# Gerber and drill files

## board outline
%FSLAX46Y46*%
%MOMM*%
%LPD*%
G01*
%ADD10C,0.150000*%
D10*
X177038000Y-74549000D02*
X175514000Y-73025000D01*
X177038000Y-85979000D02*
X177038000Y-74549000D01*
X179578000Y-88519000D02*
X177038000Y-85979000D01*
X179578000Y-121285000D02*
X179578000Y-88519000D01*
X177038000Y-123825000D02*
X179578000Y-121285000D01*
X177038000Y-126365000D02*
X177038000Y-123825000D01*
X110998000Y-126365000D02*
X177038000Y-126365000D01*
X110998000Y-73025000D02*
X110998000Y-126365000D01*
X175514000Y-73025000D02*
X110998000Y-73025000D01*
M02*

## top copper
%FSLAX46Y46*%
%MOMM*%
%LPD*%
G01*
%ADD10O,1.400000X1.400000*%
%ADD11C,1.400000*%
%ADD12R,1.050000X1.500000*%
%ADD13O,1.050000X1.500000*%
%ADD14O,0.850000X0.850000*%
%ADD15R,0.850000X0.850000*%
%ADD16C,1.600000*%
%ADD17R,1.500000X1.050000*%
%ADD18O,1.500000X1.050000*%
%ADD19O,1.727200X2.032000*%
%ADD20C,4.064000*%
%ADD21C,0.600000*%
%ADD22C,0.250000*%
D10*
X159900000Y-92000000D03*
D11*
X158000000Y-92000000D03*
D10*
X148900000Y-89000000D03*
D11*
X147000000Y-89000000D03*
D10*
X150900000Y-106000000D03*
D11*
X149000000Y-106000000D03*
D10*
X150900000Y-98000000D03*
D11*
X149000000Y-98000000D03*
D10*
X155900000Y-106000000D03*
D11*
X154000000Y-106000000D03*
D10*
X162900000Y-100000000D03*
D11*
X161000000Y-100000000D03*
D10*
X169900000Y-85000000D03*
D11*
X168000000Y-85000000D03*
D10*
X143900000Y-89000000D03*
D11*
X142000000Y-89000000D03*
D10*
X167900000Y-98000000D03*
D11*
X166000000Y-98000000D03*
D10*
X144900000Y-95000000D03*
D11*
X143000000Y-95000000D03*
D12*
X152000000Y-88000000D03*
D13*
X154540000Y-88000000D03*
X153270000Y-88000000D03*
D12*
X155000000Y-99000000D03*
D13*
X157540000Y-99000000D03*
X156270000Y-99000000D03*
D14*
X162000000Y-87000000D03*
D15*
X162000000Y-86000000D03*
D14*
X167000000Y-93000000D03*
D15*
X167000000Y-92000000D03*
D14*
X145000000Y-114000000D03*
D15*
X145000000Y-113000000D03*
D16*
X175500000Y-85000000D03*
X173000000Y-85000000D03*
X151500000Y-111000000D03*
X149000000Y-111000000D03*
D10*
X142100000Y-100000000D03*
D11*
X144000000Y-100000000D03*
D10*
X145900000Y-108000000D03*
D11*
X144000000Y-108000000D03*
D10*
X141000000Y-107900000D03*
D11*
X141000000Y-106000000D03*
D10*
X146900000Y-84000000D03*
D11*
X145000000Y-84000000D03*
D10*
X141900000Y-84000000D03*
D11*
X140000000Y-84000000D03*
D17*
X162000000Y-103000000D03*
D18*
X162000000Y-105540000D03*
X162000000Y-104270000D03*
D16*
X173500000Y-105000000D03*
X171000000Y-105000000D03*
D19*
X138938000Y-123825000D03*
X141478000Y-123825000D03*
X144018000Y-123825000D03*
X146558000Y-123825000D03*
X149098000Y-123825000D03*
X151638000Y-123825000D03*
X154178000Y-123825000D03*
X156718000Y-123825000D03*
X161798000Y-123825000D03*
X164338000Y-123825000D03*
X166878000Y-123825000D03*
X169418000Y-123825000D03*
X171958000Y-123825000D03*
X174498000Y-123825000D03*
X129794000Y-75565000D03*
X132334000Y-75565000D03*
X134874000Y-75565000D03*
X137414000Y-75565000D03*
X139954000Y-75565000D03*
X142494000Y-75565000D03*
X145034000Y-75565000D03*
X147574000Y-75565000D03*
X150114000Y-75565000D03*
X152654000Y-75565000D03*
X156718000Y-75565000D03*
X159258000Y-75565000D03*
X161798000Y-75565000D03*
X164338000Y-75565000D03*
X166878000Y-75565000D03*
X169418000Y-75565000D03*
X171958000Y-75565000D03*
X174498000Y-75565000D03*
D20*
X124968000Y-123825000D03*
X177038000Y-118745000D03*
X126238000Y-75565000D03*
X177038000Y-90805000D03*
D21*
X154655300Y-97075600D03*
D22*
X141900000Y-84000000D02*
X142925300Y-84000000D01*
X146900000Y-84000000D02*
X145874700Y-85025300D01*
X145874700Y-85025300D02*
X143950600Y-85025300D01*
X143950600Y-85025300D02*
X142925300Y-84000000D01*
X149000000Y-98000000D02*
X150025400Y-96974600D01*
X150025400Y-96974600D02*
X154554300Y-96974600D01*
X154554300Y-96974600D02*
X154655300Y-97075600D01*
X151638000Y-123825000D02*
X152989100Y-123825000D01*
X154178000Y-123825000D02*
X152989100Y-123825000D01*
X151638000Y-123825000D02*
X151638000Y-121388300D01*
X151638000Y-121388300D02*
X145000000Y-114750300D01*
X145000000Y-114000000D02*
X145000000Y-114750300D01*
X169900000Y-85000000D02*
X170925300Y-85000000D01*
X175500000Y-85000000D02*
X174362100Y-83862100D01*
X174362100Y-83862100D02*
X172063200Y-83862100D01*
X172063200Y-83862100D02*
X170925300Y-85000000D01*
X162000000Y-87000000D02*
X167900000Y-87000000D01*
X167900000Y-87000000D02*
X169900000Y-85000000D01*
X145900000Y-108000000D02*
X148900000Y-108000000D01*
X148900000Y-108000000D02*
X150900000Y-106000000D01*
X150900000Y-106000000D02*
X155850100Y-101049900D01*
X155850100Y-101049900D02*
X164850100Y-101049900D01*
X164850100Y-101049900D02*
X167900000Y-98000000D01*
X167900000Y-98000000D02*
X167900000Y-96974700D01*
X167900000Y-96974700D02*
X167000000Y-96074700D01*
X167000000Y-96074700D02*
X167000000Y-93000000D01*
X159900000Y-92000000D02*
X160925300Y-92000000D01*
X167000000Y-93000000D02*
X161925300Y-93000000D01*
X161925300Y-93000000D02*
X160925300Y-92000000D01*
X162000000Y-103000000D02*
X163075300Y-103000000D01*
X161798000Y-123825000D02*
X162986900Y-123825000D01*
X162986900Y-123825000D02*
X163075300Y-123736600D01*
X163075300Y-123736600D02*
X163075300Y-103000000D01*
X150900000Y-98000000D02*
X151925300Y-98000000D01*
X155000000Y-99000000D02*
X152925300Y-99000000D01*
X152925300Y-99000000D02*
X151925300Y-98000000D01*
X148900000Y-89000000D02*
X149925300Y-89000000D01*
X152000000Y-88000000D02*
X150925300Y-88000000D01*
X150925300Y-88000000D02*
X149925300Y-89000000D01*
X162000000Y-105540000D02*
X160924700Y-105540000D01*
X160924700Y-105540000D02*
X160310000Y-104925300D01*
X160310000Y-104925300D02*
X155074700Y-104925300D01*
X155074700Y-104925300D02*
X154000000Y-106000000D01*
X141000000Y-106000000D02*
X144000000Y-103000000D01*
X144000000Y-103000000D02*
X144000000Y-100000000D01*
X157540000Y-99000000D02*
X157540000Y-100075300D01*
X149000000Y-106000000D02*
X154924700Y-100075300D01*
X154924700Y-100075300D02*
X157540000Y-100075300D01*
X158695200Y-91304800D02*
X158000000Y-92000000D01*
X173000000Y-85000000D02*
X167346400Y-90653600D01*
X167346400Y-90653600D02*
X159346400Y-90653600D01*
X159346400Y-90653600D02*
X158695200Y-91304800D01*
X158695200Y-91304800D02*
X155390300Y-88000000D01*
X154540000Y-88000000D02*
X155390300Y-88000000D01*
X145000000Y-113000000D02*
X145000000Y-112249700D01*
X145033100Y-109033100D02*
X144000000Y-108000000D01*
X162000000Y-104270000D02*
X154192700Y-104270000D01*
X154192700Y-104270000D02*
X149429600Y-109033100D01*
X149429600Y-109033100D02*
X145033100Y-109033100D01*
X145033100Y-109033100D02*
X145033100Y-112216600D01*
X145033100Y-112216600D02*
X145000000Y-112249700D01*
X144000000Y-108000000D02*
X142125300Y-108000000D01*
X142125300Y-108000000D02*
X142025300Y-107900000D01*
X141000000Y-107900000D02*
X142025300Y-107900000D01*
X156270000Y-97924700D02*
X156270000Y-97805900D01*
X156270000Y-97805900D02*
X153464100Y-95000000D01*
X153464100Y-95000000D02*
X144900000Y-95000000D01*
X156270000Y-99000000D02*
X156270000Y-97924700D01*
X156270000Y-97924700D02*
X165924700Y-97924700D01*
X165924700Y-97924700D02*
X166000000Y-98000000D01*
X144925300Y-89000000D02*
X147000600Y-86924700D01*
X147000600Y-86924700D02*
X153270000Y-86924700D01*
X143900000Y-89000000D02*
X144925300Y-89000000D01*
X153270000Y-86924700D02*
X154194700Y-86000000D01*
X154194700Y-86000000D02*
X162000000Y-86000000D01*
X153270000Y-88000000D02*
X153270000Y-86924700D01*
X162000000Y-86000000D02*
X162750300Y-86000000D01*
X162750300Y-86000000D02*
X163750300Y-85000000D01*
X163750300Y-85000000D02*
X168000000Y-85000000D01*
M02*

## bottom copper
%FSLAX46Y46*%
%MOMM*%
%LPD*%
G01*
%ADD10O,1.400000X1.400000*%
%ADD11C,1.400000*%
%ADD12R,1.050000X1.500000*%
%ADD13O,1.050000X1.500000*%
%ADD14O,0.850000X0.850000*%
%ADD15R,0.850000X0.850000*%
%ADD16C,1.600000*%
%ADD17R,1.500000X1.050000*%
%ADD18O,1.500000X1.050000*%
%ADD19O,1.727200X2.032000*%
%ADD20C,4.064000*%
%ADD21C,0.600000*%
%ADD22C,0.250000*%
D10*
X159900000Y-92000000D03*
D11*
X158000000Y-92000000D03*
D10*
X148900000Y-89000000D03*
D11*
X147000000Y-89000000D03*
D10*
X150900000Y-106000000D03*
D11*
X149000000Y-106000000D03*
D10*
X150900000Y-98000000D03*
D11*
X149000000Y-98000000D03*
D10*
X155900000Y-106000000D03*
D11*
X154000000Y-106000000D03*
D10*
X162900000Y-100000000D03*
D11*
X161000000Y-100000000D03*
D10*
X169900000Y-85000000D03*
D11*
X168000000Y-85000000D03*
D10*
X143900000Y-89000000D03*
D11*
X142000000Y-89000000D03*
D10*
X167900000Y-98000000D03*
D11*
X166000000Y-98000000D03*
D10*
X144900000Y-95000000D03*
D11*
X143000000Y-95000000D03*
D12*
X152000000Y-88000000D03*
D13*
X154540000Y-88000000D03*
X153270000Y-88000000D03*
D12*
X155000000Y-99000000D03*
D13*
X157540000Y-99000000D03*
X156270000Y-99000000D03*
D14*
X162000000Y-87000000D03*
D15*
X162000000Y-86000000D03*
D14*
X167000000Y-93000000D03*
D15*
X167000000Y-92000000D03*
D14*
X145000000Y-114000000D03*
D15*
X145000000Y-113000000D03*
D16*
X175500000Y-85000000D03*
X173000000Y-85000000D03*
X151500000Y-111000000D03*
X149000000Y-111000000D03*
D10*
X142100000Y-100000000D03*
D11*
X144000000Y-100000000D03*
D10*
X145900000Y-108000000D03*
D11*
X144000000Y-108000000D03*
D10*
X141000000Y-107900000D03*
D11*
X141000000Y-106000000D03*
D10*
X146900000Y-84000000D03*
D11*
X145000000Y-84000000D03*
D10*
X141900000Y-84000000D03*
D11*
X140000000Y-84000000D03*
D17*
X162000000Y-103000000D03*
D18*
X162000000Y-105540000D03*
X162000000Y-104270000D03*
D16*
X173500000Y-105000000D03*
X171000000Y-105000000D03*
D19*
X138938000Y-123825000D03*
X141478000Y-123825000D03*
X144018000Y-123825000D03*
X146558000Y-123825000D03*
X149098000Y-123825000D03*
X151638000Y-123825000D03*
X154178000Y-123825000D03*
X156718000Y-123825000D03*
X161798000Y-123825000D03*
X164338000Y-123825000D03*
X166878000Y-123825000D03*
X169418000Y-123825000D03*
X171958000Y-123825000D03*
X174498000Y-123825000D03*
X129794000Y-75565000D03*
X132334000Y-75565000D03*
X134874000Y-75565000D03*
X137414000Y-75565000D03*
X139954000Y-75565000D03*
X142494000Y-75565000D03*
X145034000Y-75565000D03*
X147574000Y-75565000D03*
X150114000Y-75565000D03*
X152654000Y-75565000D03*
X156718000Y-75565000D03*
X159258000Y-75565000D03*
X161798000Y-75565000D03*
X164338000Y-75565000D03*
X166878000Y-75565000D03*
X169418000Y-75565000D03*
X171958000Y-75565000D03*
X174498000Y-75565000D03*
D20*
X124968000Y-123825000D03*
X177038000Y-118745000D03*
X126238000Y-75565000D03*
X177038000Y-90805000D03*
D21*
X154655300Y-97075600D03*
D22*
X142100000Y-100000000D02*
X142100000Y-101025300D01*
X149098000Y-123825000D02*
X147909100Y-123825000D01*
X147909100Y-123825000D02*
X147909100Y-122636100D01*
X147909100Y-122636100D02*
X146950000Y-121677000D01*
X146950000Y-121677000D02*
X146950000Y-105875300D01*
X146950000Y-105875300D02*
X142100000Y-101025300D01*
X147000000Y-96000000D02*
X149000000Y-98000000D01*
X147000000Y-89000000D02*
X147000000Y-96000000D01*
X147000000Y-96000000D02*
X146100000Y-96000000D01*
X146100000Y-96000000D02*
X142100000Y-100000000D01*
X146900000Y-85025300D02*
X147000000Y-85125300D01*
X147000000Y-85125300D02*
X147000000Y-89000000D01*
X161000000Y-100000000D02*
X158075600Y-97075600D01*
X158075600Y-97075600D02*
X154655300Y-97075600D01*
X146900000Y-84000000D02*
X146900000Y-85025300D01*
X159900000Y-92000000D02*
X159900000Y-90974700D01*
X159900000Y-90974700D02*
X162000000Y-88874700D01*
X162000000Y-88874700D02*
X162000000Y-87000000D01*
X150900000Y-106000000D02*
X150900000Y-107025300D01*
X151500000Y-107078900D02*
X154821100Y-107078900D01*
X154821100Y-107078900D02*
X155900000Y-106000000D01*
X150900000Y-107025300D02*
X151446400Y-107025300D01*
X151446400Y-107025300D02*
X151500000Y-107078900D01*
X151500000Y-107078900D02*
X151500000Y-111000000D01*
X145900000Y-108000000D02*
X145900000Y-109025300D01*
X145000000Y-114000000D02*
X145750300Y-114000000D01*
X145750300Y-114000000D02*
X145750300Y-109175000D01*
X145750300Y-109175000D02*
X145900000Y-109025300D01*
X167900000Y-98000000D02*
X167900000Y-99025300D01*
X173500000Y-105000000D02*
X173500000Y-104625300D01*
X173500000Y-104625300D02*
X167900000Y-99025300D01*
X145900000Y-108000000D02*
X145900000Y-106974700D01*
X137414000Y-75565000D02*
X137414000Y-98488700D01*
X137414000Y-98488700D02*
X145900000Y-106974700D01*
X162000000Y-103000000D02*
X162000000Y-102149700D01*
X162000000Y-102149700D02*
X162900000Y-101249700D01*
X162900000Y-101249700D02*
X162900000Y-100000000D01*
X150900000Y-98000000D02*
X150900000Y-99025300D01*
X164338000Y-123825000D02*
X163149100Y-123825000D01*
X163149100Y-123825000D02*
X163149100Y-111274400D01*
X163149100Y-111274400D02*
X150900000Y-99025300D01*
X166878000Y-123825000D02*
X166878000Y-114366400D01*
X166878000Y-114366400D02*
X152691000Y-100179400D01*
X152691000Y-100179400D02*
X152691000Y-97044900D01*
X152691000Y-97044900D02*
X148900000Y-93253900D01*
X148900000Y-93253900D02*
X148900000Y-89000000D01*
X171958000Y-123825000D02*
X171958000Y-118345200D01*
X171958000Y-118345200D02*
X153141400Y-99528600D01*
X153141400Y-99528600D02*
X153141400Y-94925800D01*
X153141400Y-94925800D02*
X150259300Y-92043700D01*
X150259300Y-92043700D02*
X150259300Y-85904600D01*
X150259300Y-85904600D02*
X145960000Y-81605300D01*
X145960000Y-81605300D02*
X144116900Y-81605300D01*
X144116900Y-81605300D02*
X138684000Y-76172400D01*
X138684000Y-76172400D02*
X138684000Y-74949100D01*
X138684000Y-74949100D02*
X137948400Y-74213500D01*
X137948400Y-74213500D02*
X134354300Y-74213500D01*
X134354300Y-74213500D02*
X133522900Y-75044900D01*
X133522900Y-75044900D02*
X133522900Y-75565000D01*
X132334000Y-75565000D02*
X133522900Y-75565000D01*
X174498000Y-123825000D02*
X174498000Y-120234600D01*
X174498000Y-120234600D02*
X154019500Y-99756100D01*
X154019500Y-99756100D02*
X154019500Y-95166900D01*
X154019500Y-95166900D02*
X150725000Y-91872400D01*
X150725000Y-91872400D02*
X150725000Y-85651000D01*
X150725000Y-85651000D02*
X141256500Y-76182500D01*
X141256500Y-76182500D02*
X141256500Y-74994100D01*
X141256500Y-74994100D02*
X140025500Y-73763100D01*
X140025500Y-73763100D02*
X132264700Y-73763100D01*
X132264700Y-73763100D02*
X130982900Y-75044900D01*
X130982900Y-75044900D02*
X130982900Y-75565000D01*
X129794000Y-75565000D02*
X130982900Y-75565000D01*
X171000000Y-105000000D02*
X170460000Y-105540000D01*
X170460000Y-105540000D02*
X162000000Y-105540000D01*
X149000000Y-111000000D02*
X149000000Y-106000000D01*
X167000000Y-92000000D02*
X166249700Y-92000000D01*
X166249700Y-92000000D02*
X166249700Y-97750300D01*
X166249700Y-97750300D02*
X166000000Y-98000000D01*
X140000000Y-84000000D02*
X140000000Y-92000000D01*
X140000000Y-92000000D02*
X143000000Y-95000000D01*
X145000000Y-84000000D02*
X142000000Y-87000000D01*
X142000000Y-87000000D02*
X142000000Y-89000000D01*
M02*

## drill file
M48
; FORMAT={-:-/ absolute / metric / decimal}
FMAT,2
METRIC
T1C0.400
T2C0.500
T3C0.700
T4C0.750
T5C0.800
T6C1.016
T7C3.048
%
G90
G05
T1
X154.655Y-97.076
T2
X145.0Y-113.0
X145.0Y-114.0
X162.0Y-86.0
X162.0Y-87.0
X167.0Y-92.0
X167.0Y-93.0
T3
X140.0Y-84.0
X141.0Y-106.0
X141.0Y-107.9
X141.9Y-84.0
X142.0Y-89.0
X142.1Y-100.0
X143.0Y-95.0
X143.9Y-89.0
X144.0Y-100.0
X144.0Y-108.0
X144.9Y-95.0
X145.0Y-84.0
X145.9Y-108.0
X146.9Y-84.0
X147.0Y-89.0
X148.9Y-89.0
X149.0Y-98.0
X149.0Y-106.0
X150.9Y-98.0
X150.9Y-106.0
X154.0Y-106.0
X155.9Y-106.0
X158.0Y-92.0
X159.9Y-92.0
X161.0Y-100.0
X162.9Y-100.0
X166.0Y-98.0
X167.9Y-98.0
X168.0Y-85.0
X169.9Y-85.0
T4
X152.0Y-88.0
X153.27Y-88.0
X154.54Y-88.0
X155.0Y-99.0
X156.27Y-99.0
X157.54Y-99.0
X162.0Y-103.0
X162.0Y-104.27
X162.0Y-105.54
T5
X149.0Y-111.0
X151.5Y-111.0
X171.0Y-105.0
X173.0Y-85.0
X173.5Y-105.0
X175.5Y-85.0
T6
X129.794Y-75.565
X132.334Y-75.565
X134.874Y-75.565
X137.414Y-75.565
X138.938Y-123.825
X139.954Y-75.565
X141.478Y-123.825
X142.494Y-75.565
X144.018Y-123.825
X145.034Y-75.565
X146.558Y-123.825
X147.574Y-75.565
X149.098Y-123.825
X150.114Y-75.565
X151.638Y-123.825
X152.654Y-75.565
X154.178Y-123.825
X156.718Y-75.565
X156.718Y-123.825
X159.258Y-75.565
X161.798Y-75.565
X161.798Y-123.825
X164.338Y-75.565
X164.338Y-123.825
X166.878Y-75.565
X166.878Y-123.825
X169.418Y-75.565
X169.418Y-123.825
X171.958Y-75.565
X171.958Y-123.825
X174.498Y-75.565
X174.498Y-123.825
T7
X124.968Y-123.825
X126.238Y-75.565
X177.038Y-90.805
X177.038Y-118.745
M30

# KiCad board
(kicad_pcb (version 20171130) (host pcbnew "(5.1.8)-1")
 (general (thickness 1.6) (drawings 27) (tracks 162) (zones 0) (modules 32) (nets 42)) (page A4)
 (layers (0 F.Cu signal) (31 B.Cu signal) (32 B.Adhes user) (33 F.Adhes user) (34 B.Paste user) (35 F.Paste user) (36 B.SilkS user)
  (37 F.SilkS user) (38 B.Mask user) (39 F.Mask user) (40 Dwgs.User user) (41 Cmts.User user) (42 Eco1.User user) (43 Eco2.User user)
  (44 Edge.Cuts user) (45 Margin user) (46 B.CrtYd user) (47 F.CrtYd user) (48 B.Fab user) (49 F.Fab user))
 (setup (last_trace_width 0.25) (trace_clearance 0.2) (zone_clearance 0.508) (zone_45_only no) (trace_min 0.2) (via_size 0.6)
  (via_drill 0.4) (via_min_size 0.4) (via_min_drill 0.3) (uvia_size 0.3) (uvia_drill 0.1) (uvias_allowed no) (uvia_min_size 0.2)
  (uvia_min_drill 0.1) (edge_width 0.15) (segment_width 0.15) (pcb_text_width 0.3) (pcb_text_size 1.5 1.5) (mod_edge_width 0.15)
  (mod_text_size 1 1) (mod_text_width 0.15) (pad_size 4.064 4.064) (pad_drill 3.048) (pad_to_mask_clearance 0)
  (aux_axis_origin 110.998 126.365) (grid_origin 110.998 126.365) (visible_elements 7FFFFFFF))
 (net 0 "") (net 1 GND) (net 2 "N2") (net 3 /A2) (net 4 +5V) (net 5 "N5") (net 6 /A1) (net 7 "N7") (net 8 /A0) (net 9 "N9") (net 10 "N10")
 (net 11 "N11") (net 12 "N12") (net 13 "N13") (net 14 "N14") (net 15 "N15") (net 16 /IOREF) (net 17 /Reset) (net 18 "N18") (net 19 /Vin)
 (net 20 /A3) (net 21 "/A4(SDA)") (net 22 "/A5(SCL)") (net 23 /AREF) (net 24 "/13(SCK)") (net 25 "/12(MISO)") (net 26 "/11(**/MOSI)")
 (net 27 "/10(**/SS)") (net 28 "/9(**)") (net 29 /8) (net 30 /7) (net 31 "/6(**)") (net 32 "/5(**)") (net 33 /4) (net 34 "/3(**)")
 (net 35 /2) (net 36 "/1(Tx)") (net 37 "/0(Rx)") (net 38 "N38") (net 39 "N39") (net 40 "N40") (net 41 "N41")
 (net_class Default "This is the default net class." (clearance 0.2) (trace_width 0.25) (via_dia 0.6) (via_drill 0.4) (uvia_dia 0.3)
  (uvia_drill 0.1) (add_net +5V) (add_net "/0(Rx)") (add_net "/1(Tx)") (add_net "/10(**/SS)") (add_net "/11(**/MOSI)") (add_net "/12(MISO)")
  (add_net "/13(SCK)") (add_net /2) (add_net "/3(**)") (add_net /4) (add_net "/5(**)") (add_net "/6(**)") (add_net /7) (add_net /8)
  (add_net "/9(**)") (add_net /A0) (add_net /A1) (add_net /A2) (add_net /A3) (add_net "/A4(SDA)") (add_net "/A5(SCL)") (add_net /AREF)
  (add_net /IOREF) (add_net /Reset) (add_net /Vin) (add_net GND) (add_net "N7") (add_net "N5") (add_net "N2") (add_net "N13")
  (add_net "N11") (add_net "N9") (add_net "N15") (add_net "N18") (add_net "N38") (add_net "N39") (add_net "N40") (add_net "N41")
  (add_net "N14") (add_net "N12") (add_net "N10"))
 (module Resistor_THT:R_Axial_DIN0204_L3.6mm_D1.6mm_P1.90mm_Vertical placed (layer F.Cu) (at 158 92)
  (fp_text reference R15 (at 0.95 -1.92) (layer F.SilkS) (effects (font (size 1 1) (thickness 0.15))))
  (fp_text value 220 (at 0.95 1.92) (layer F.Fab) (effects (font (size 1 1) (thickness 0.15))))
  (pad 2 thru_hole oval (at 1.9 0) (size 1.4 1.4) (drill 0.7) (layers *.Cu *.Mask) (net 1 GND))
  (pad 1 thru_hole circle (at 0 0) (size 1.4 1.4) (drill 0.7) (layers *.Cu *.Mask) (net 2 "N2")))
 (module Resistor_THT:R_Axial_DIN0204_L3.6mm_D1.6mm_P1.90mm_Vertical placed (layer F.Cu) (at 147 89)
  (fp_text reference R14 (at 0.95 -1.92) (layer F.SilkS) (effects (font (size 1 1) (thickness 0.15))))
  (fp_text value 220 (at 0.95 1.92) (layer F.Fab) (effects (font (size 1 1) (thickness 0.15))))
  (pad 2 thru_hole oval (at 1.9 0) (size 1.4 1.4) (drill 0.7) (layers *.Cu *.Mask) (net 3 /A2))
  (pad 1 thru_hole circle (at 0 0) (size 1.4 1.4) (drill 0.7) (layers *.Cu *.Mask) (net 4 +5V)))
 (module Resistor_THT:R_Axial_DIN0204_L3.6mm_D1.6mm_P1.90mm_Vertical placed (layer F.Cu) (at 149 106)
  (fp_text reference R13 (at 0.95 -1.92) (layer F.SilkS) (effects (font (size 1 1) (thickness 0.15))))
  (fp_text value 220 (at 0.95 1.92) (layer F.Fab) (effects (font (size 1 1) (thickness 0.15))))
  (pad 2 thru_hole oval (at 1.9 0) (size 1.4 1.4) (drill 0.7) (layers *.Cu *.Mask) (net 1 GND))
  (pad 1 thru_hole circle (at 0 0) (size 1.4 1.4) (drill 0.7) (layers *.Cu *.Mask) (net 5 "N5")))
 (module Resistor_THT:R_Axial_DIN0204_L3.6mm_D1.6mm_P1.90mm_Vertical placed (layer F.Cu) (at 149 98)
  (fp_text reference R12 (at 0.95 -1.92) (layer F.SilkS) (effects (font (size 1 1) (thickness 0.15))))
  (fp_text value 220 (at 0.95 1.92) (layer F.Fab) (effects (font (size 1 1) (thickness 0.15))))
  (pad 2 thru_hole oval (at 1.9 0) (size 1.4 1.4) (drill 0.7) (layers *.Cu *.Mask) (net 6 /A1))
  (pad 1 thru_hole circle (at 0 0) (size 1.4 1.4) (drill 0.7) (layers *.Cu *.Mask) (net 4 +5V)))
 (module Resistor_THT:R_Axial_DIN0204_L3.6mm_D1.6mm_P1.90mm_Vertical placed (layer F.Cu) (at 154 106)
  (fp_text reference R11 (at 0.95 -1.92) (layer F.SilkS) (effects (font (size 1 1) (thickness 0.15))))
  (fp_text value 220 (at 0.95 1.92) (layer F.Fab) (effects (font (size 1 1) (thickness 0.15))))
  (pad 2 thru_hole oval (at 1.9 0) (size 1.4 1.4) (drill 0.7) (layers *.Cu *.Mask) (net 1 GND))
  (pad 1 thru_hole circle (at 0 0) (size 1.4 1.4) (drill 0.7) (layers *.Cu *.Mask) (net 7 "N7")))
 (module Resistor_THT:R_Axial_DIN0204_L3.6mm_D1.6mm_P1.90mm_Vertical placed (layer F.Cu) (at 161 100)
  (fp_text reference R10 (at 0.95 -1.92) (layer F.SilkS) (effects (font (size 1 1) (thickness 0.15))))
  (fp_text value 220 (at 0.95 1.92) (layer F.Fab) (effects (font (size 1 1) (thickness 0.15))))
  (pad 2 thru_hole oval (at 1.9 0) (size 1.4 1.4) (drill 0.7) (layers *.Cu *.Mask) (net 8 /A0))
  (pad 1 thru_hole circle (at 0 0) (size 1.4 1.4) (drill 0.7) (layers *.Cu *.Mask) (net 4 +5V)))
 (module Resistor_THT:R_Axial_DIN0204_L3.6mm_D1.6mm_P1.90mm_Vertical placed (layer F.Cu) (at 168 85)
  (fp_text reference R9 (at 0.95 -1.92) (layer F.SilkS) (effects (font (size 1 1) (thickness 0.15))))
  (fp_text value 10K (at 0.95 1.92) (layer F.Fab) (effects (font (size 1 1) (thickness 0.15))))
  (pad 2 thru_hole oval (at 1.9 0) (size 1.4 1.4) (drill 0.7) (layers *.Cu *.Mask) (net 1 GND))
  (pad 1 thru_hole circle (at 0 0) (size 1.4 1.4) (drill 0.7) (layers *.Cu *.Mask) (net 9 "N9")))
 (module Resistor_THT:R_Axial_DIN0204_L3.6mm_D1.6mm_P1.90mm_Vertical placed (layer F.Cu) (at 142 89)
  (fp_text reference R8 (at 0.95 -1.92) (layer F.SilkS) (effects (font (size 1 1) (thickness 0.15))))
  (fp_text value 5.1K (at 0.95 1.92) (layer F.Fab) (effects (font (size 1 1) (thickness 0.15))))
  (pad 2 thru_hole oval (at 1.9 0) (size 1.4 1.4) (drill 0.7) (layers *.Cu *.Mask) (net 9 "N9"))
  (pad 1 thru_hole circle (at 0 0) (size 1.4 1.4) (drill 0.7) (layers *.Cu *.Mask) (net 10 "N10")))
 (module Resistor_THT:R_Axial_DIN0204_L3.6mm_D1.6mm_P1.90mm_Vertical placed (layer F.Cu) (at 166 98)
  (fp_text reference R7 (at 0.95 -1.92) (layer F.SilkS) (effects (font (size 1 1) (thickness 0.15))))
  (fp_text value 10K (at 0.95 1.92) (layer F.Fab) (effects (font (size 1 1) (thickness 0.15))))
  (pad 2 thru_hole oval (at 1.9 0) (size 1.4 1.4) (drill 0.7) (layers *.Cu *.Mask) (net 1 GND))
  (pad 1 thru_hole circle (at 0 0) (size 1.4 1.4) (drill 0.7) (layers *.Cu *.Mask) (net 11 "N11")))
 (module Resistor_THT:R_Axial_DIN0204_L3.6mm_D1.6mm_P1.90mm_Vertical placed (layer F.Cu) (at 143 95)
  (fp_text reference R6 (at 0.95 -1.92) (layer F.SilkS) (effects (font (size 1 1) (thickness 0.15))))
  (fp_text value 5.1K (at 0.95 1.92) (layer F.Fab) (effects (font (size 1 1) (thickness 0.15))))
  (pad 2 thru_hole oval (at 1.9 0) (size 1.4 1.4) (drill 0.7) (layers *.Cu *.Mask) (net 11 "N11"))
  (pad 1 thru_hole circle (at 0 0) (size 1.4 1.4) (drill 0.7) (layers *.Cu *.Mask) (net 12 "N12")))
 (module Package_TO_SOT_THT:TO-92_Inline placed (layer F.Cu) (at 152 88)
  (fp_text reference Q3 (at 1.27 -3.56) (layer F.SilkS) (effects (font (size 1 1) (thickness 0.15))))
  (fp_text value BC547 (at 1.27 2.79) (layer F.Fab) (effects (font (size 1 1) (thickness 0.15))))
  (pad 1 thru_hole rect (at 0 0) (size 1.05 1.5) (drill 0.75) (layers *.Cu *.Mask) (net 3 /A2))
  (pad 3 thru_hole oval (at 2.54 0) (size 1.05 1.5) (drill 0.75) (layers *.Cu *.Mask) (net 2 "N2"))
  (pad 2 thru_hole oval (at 1.27 0) (size 1.05 1.5) (drill 0.75) (layers *.Cu *.Mask) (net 9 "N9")))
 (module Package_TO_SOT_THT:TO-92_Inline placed (layer F.Cu) (at 155 99)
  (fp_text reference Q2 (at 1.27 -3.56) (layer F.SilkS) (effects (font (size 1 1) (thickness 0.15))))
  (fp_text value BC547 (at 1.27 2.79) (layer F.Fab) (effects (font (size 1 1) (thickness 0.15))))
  (pad 1 thru_hole rect (at 0 0) (size 1.05 1.5) (drill 0.75) (layers *.Cu *.Mask) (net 6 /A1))
  (pad 3 thru_hole oval (at 2.54 0) (size 1.05 1.5) (drill 0.75) (layers *.Cu *.Mask) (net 5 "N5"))
  (pad 2 thru_hole oval (at 1.27 0) (size 1.05 1.5) (drill 0.75) (layers *.Cu *.Mask) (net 11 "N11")))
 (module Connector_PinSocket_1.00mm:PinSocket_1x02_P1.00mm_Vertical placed (layer F.Cu) (at 162 86)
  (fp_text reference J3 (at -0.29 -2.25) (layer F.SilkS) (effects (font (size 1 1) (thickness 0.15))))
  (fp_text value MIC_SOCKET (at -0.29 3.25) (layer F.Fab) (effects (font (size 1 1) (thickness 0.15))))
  (pad 2 thru_hole oval (at 0 1) (size 0.85 0.85) (drill 0.5) (layers *.Cu *.Mask) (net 1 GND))
  (pad 1 thru_hole rect (at 0 0) (size 0.85 0.85) (drill 0.5) (layers *.Cu *.Mask) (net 9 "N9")))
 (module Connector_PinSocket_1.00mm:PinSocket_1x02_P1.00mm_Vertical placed (layer F.Cu) (at 167 92)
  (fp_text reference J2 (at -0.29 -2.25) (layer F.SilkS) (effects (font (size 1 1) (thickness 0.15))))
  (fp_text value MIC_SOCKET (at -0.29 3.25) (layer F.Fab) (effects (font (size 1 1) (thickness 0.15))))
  (pad 2 thru_hole oval (at 0 1) (size 0.85 0.85) (drill 0.5) (layers *.Cu *.Mask) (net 1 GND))
  (pad 1 thru_hole rect (at 0 0) (size 0.85 0.85) (drill 0.5) (layers *.Cu *.Mask) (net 11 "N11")))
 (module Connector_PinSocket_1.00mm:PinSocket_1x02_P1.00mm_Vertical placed (layer F.Cu) (at 145 113)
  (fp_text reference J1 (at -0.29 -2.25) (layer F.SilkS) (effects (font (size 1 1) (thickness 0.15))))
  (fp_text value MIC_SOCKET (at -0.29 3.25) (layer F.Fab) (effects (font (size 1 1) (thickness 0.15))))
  (pad 2 thru_hole oval (at 0 1) (size 0.85 0.85) (drill 0.5) (layers *.Cu *.Mask) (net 1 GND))
  (pad 1 thru_hole rect (at 0 0) (size 0.85 0.85) (drill 0.5) (layers *.Cu *.Mask) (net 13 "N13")))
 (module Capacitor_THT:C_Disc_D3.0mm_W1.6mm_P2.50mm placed (layer F.Cu) (at 173 85)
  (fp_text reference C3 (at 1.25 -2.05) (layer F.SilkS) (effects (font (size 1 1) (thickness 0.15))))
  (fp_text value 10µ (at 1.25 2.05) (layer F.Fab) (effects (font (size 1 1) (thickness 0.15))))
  (pad 2 thru_hole circle (at 2.5 0) (size 1.6 1.6) (drill 0.8) (layers *.Cu *.Mask) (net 1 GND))
  (pad 1 thru_hole circle (at 0 0) (size 1.6 1.6) (drill 0.8) (layers *.Cu *.Mask) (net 2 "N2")))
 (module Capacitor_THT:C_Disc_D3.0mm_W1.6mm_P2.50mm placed (layer F.Cu) (at 149 111)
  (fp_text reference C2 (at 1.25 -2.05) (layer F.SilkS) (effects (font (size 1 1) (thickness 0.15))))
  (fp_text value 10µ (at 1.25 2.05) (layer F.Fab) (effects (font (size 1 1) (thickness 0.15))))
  (pad 2 thru_hole circle (at 2.5 0) (size 1.6 1.6) (drill 0.8) (layers *.Cu *.Mask) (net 1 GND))
  (pad 1 thru_hole circle (at 0 0) (size 1.6 1.6) (drill 0.8) (layers *.Cu *.Mask) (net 5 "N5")))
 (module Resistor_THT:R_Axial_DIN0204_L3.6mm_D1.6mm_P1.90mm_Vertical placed (layer F.Cu) (at 144 100 180)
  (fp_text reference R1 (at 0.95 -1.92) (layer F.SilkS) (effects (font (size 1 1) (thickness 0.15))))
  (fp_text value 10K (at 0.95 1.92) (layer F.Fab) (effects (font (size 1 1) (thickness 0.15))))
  (pad 2 thru_hole oval (at 1.9 0 180) (size 1.4 1.4) (drill 0.7) (layers *.Cu *.Mask) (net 4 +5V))
  (pad 1 thru_hole circle (at 0 0 180) (size 1.4 1.4) (drill 0.7) (layers *.Cu *.Mask) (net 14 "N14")))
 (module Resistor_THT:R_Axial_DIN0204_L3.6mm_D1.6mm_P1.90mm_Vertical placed (layer F.Cu) (at 144 108)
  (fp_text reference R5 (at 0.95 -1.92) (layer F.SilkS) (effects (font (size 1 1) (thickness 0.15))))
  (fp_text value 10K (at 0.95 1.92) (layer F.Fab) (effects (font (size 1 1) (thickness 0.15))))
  (pad 2 thru_hole oval (at 1.9 0) (size 1.4 1.4) (drill 0.7) (layers *.Cu *.Mask) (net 1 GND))
  (pad 1 thru_hole circle (at 0 0) (size 1.4 1.4) (drill 0.7) (layers *.Cu *.Mask) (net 13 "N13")))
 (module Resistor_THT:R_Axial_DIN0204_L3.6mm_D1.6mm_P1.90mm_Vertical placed (layer F.Cu) (at 141 106 270)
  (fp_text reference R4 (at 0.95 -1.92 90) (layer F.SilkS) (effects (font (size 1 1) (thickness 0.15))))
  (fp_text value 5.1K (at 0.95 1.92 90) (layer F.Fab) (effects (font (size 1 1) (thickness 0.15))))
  (pad 2 thru_hole oval (at 1.9 0 270) (size 1.4 1.4) (drill 0.7) (layers *.Cu *.Mask) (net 13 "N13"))
  (pad 1 thru_hole circle (at 0 0 270) (size 1.4 1.4) (drill 0.7) (layers *.Cu *.Mask) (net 14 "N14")))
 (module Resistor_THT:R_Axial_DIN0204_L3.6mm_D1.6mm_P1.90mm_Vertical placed (layer F.Cu) (at 145 84)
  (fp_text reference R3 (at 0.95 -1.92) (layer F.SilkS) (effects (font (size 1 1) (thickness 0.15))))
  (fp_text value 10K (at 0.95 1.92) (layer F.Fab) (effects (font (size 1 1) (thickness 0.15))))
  (pad 2 thru_hole oval (at 1.9 0) (size 1.4 1.4) (drill 0.7) (layers *.Cu *.Mask) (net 4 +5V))
  (pad 1 thru_hole circle (at 0 0) (size 1.4 1.4) (drill 0.7) (layers *.Cu *.Mask) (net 10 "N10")))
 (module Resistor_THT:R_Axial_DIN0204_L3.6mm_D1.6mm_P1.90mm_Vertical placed (layer F.Cu) (at 140 84)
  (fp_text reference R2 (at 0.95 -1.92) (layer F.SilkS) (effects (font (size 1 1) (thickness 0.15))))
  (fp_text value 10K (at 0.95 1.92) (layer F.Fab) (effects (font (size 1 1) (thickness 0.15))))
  (pad 2 thru_hole oval (at 1.9 0) (size 1.4 1.4) (drill 0.7) (layers *.Cu *.Mask) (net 4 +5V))
  (pad 1 thru_hole circle (at 0 0) (size 1.4 1.4) (drill 0.7) (layers *.Cu *.Mask) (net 12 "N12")))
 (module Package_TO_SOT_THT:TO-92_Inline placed (layer F.Cu) (at 162 103 270)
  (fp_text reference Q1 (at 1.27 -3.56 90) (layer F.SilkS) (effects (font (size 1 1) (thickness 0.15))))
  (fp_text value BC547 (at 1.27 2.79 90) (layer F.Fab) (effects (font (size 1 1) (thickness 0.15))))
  (pad 1 thru_hole rect (at 0 0 270) (size 1.05 1.5) (drill 0.75) (layers *.Cu *.Mask) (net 8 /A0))
  (pad 3 thru_hole oval (at 2.54 0 270) (size 1.05 1.5) (drill 0.75) (layers *.Cu *.Mask) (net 7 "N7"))
  (pad 2 thru_hole oval (at 1.27 0 270) (size 1.05 1.5) (drill 0.75) (layers *.Cu *.Mask) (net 13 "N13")))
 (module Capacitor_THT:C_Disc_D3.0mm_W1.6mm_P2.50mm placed (layer F.Cu) (at 171 105)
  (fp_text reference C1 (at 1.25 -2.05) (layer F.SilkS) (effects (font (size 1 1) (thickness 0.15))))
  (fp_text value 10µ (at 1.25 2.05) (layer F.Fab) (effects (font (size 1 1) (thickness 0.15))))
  (pad 2 thru_hole circle (at 2.5 0) (size 1.6 1.6) (drill 0.8) (layers *.Cu *.Mask) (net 1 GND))
  (pad 1 thru_hole circle (at 0 0) (size 1.6 1.6) (drill 0.8) (layers *.Cu *.Mask) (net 7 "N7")))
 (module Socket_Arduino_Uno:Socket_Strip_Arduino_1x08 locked (layer F.Cu) (at 138.938 123.825)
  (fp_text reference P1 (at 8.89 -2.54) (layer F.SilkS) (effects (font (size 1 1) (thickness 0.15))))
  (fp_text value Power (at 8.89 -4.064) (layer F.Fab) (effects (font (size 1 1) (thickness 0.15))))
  (pad 1 thru_hole oval (at 0 0) (size 1.7272 2.032) (drill 1.016) (layers *.Cu *.Mask F.SilkS) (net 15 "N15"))
  (pad 2 thru_hole oval (at 2.54 0) (size 1.7272 2.032) (drill 1.016) (layers *.Cu *.Mask F.SilkS) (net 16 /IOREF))
  (pad 3 thru_hole oval (at 5.08 0) (size 1.7272 2.032) (drill 1.016) (layers *.Cu *.Mask F.SilkS) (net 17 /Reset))
  (pad 4 thru_hole oval (at 7.62 0) (size 1.7272 2.032) (drill 1.016) (layers *.Cu *.Mask F.SilkS) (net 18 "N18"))
  (pad 5 thru_hole oval (at 10.16 0) (size 1.7272 2.032) (drill 1.016) (layers *.Cu *.Mask F.SilkS) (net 4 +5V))
  (pad 6 thru_hole oval (at 12.7 0) (size 1.7272 2.032) (drill 1.016) (layers *.Cu *.Mask F.SilkS) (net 1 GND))
  (pad 7 thru_hole oval (at 15.24 0) (size 1.7272 2.032) (drill 1.016) (layers *.Cu *.Mask F.SilkS) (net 1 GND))
  (pad 8 thru_hole oval (at 17.78 0) (size 1.7272 2.032) (drill 1.016) (layers *.Cu *.Mask F.SilkS) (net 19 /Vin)))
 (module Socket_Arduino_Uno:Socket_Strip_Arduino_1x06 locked (layer F.Cu) (at 161.798 123.825)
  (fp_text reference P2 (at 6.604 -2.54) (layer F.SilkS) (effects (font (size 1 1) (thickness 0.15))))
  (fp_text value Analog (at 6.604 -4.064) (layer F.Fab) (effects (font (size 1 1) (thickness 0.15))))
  (pad 1 thru_hole oval (at 0 0) (size 1.7272 2.032) (drill 1.016) (layers *.Cu *.Mask F.SilkS) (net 8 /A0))
  (pad 2 thru_hole oval (at 2.54 0) (size 1.7272 2.032) (drill 1.016) (layers *.Cu *.Mask F.SilkS) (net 6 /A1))
  (pad 3 thru_hole oval (at 5.08 0) (size 1.7272 2.032) (drill 1.016) (layers *.Cu *.Mask F.SilkS) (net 3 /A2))
  (pad 4 thru_hole oval (at 7.62 0) (size 1.7272 2.032) (drill 1.016) (layers *.Cu *.Mask F.SilkS) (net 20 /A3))
  (pad 5 thru_hole oval (at 10.16 0) (size 1.7272 2.032) (drill 1.016) (layers *.Cu *.Mask F.SilkS) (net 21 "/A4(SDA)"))
  (pad 6 thru_hole oval (at 12.7 0) (size 1.7272 2.032) (drill 1.016) (layers *.Cu *.Mask F.SilkS) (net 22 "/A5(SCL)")))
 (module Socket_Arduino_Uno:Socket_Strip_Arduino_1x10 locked (layer F.Cu) (at 129.794 75.565)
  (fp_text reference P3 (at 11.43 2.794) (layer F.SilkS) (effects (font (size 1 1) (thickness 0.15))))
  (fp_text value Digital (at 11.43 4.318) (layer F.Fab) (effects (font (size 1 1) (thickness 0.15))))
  (pad 1 thru_hole oval (at 0 0) (size 1.7272 2.032) (drill 1.016) (layers *.Cu *.Mask F.SilkS) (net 22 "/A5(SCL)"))
  (pad 2 thru_hole oval (at 2.54 0) (size 1.7272 2.032) (drill 1.016) (layers *.Cu *.Mask F.SilkS) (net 21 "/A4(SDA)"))
  (pad 3 thru_hole oval (at 5.08 0) (size 1.7272 2.032) (drill 1.016) (layers *.Cu *.Mask F.SilkS) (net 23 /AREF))
  (pad 4 thru_hole oval (at 7.62 0) (size 1.7272 2.032) (drill 1.016) (layers *.Cu *.Mask F.SilkS) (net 1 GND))
  (pad 5 thru_hole oval (at 10.16 0) (size 1.7272 2.032) (drill 1.016) (layers *.Cu *.Mask F.SilkS) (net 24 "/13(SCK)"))
  (pad 6 thru_hole oval (at 12.7 0) (size 1.7272 2.032) (drill 1.016) (layers *.Cu *.Mask F.SilkS) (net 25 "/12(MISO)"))
  (pad 7 thru_hole oval (at 15.24 0) (size 1.7272 2.032) (drill 1.016) (layers *.Cu *.Mask F.SilkS) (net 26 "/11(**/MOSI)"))
  (pad 8 thru_hole oval (at 17.78 0) (size 1.7272 2.032) (drill 1.016) (layers *.Cu *.Mask F.SilkS) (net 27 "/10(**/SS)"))
  (pad 9 thru_hole oval (at 20.32 0) (size 1.7272 2.032) (drill 1.016) (layers *.Cu *.Mask F.SilkS) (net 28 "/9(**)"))
  (pad 10 thru_hole oval (at 22.86 0) (size 1.7272 2.032) (drill 1.016) (layers *.Cu *.Mask F.SilkS) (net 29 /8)))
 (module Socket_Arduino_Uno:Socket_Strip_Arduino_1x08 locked (layer F.Cu) (at 156.718 75.565)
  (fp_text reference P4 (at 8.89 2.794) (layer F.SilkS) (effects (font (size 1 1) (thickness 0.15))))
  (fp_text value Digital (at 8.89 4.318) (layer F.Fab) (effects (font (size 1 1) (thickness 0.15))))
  (pad 1 thru_hole oval (at 0 0) (size 1.7272 2.032) (drill 1.016) (layers *.Cu *.Mask F.SilkS) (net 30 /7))
  (pad 2 thru_hole oval (at 2.54 0) (size 1.7272 2.032) (drill 1.016) (layers *.Cu *.Mask F.SilkS) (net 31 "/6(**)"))
  (pad 3 thru_hole oval (at 5.08 0) (size 1.7272 2.032) (drill 1.016) (layers *.Cu *.Mask F.SilkS) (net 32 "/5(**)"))
  (pad 4 thru_hole oval (at 7.62 0) (size 1.7272 2.032) (drill 1.016) (layers *.Cu *.Mask F.SilkS) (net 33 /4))
  (pad 5 thru_hole oval (at 10.16 0) (size 1.7272 2.032) (drill 1.016) (layers *.Cu *.Mask F.SilkS) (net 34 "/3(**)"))
  (pad 6 thru_hole oval (at 12.7 0) (size 1.7272 2.032) (drill 1.016) (layers *.Cu *.Mask F.SilkS) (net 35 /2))
  (pad 7 thru_hole oval (at 15.24 0) (size 1.7272 2.032) (drill 1.016) (layers *.Cu *.Mask F.SilkS) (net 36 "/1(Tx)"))
  (pad 8 thru_hole oval (at 17.78 0) (size 1.7272 2.032) (drill 1.016) (layers *.Cu *.Mask F.SilkS) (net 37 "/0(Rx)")))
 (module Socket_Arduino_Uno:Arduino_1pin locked (layer F.Cu) (at 124.968 123.825)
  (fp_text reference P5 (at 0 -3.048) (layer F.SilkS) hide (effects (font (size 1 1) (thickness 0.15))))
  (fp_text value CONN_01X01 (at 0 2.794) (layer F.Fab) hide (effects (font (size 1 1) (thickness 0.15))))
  (pad 1 thru_hole circle (at 0 0) (size 4.064 4.064) (drill 3.048) (layers *.Cu *.Mask F.SilkS) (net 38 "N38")))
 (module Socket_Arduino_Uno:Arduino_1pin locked (layer F.Cu) (at 177.038 118.745)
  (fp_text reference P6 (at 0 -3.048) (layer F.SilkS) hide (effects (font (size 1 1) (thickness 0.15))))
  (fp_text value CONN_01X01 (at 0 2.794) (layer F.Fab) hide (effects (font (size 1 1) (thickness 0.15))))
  (pad 1 thru_hole circle (at 0 0) (size 4.064 4.064) (drill 3.048) (layers *.Cu *.Mask F.SilkS) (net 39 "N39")))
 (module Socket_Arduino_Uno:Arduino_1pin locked (layer F.Cu) (at 126.238 75.565)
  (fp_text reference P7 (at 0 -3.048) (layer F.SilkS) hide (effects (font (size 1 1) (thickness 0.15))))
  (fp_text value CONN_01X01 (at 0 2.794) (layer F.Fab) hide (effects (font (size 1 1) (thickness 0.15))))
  (pad 1 thru_hole circle (at 0 0) (size 4.064 4.064) (drill 3.048) (layers *.Cu *.Mask F.SilkS) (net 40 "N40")))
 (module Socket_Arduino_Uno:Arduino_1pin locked (layer F.Cu) (at 177.038 90.805)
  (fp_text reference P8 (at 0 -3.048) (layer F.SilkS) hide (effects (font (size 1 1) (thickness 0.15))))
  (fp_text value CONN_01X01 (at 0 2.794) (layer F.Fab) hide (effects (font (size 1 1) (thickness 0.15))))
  (pad 1 thru_hole circle (at 0 0) (size 4.064 4.064) (drill 3.048) (layers *.Cu *.Mask F.SilkS) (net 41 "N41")))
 (gr_line (start 177.038 74.549) (end 175.514 73.025) (angle 90) (layer Edge.Cuts) (width 0.15))
 (gr_line (start 177.038 85.979) (end 177.038 74.549) (angle 90) (layer Edge.Cuts) (width 0.15))
 (gr_line (start 179.578 88.519) (end 177.038 85.979) (angle 90) (layer Edge.Cuts) (width 0.15))
 (gr_line (start 179.578 121.285) (end 179.578 88.519) (angle 90) (layer Edge.Cuts) (width 0.15))
 (gr_line (start 177.038 123.825) (end 179.578 121.285) (angle 90) (layer Edge.Cuts) (width 0.15))
 (gr_line (start 177.038 126.365) (end 177.038 123.825) (angle 90) (layer Edge.Cuts) (width 0.15))
 (gr_line (start 110.998 126.365) (end 177.038 126.365) (angle 90) (layer Edge.Cuts) (width 0.15))
 (gr_line (start 110.998 73.025) (end 110.998 126.365) (angle 90) (layer Edge.Cuts) (width 0.15))
 (gr_line (start 175.514 73.025) (end 110.998 73.025) (angle 90) (layer Edge.Cuts) (width 0.15))
 (segment (start 142.1 100) (end 142.1 101.0253) (width 0.25) (layer B.Cu) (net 4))
 (segment (start 149.098 123.825) (end 147.9091 123.825) (width 0.25) (layer B.Cu) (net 4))
 (segment (start 147.9091 123.825) (end 147.9091 122.6361) (width 0.25) (layer B.Cu) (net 4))
 (segment (start 147.9091 122.6361) (end 146.95 121.677) (width 0.25) (layer B.Cu) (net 4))
 (segment (start 146.95 121.677) (end 146.95 105.8753) (width 0.25) (layer B.Cu) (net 4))
 (segment (start 146.95 105.8753) (end 142.1 101.0253) (width 0.25) (layer B.Cu) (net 4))
 (segment (start 147 96) (end 149 98) (width 0.25) (layer B.Cu) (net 4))
 (segment (start 147 89) (end 147 96) (width 0.25) (layer B.Cu) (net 4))
 (segment (start 147 96) (end 146.1 96) (width 0.25) (layer B.Cu) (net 4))
 (segment (start 146.1 96) (end 142.1 100) (width 0.25) (layer B.Cu) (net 4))
 (segment (start 146.9 85.0253) (end 147 85.1253) (width 0.25) (layer B.Cu) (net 4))
 (segment (start 147 85.1253) (end 147 89) (width 0.25) (layer B.Cu) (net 4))
 (segment (start 141.9 84) (end 142.9253 84) (width 0.25) (layer F.Cu) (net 4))
 (segment (start 146.9 84) (end 145.8747 85.0253) (width 0.25) (layer F.Cu) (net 4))
 (segment (start 145.8747 85.0253) (end 143.9506 85.0253) (width 0.25) (layer F.Cu) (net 4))
 (segment (start 143.9506 85.0253) (end 142.9253 84) (width 0.25) (layer F.Cu) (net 4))
 (segment (start 149 98) (end 150.0254 96.9746) (width 0.25) (layer F.Cu) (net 4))
 (segment (start 150.0254 96.9746) (end 154.5543 96.9746) (width 0.25) (layer F.Cu) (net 4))
 (segment (start 154.5543 96.9746) (end 154.6553 97.0756) (width 0.25) (layer F.Cu) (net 4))
 (segment (start 161 100) (end 158.0756 97.0756) (width 0.25) (layer B.Cu) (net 4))
 (segment (start 158.0756 97.0756) (end 154.6553 97.0756) (width 0.25) (layer B.Cu) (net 4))
 (segment (start 146.9 84) (end 146.9 85.0253) (width 0.25) (layer B.Cu) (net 4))
 (via (at 154.6553 97.0756) (size 0.6) (layers F.Cu B.Cu) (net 4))
 (segment (start 159.9 92) (end 159.9 90.9747) (width 0.25) (layer B.Cu) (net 1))
 (segment (start 159.9 90.9747) (end 162 88.8747) (width 0.25) (layer B.Cu) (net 1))
 (segment (start 162 88.8747) (end 162 87) (width 0.25) (layer B.Cu) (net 1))
 (segment (start 150.9 106) (end 150.9 107.0253) (width 0.25) (layer B.Cu) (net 1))
 (segment (start 151.5 107.0789) (end 154.8211 107.0789) (width 0.25) (layer B.Cu) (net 1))
 (segment (start 154.8211 107.0789) (end 155.9 106) (width 0.25) (layer B.Cu) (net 1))
 (segment (start 150.9 107.0253) (end 151.4464 107.0253) (width 0.25) (layer B.Cu) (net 1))
 (segment (start 151.4464 107.0253) (end 151.5 107.0789) (width 0.25) (layer B.Cu) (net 1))
 (segment (start 151.5 107.0789) (end 151.5 111) (width 0.25) (layer B.Cu) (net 1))
 (segment (start 151.638 123.825) (end 152.9891 123.825) (width 0.25) (layer F.Cu) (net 1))
 (segment (start 154.178 123.825) (end 152.9891 123.825) (width 0.25) (layer F.Cu) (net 1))
 (segment (start 151.638 123.825) (end 151.638 121.3883) (width 0.25) (layer F.Cu) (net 1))
 (segment (start 151.638 121.3883) (end 145 114.7503) (width 0.25) (layer F.Cu) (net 1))
 (segment (start 145 114) (end 145 114.7503) (width 0.25) (layer F.Cu) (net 1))
 (segment (start 169.9 85) (end 170.9253 85) (width 0.25) (layer F.Cu) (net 1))
 (segment (start 175.5 85) (end 174.3621 83.8621) (width 0.25) (layer F.Cu) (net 1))
 (segment (start 174.3621 83.8621) (end 172.0632 83.8621) (width 0.25) (layer F.Cu) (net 1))
 (segment (start 172.0632 83.8621) (end 170.9253 85) (width 0.25) (layer F.Cu) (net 1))
 (segment (start 162 87) (end 167.9 87) (width 0.25) (layer F.Cu) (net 1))
 (segment (start 167.9 87) (end 169.9 85) (width 0.25) (layer F.Cu) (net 1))
 (segment (start 145.9 108) (end 148.9 108) (width 0.25) (layer F.Cu) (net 1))
 (segment (start 148.9 108) (end 150.9 106) (width 0.25) (layer F.Cu) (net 1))
 (segment (start 150.9 106) (end 155.8501 101.0499) (width 0.25) (layer F.Cu) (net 1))
 (segment (start 155.8501 101.0499) (end 164.8501 101.0499) (width 0.25) (layer F.Cu) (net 1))
 (segment (start 164.8501 101.0499) (end 167.9 98) (width 0.25) (layer F.Cu) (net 1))
 (segment (start 167.9 98) (end 167.9 96.9747) (width 0.25) (layer F.Cu) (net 1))
 (segment (start 167.9 96.9747) (end 167 96.0747) (width 0.25) (layer F.Cu) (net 1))
 (segment (start 167 96.0747) (end 167 93) (width 0.25) (layer F.Cu) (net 1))
 (segment (start 159.9 92) (end 160.9253 92) (width 0.25) (layer F.Cu) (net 1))
 (segment (start 167 93) (end 161.9253 93) (width 0.25) (layer F.Cu) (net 1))
 (segment (start 161.9253 93) (end 160.9253 92) (width 0.25) (layer F.Cu) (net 1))
 (segment (start 145.9 108) (end 145.9 109.0253) (width 0.25) (layer B.Cu) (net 1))
 (segment (start 145 114) (end 145.7503 114) (width 0.25) (layer B.Cu) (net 1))
 (segment (start 145.7503 114) (end 145.7503 109.175) (width 0.25) (layer B.Cu) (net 1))
 (segment (start 145.7503 109.175) (end 145.9 109.0253) (width 0.25) (layer B.Cu) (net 1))
 (segment (start 167.9 98) (end 167.9 99.0253) (width 0.25) (layer B.Cu) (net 1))
 (segment (start 173.5 105) (end 173.5 104.6253) (width 0.25) (layer B.Cu) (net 1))
 (segment (start 173.5 104.6253) (end 167.9 99.0253) (width 0.25) (layer B.Cu) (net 1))
 (segment (start 145.9 108) (end 145.9 106.9747) (width 0.25) (layer B.Cu) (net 1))
 (segment (start 137.414 75.565) (end 137.414 98.4887) (width 0.25) (layer B.Cu) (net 1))
 (segment (start 137.414 98.4887) (end 145.9 106.9747) (width 0.25) (layer B.Cu) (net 1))
 (segment (start 162 103) (end 162 102.1497) (width 0.25) (layer B.Cu) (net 8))
 (segment (start 162 102.1497) (end 162.9 101.2497) (width 0.25) (layer B.Cu) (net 8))
 (segment (start 162.9 101.2497) (end 162.9 100) (width 0.25) (layer B.Cu) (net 8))
 (segment (start 162 103) (end 163.0753 103) (width 0.25) (layer F.Cu) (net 8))
 (segment (start 161.798 123.825) (end 162.9869 123.825) (width 0.25) (layer F.Cu) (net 8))
 (segment (start 162.9869 123.825) (end 163.0753 123.7366) (width 0.25) (layer F.Cu) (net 8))
 (segment (start 163.0753 123.7366) (end 163.0753 103) (width 0.25) (layer F.Cu) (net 8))
 (segment (start 150.9 98) (end 151.9253 98) (width 0.25) (layer F.Cu) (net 6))
 (segment (start 155 99) (end 152.9253 99) (width 0.25) (layer F.Cu) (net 6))
 (segment (start 152.9253 99) (end 151.9253 98) (width 0.25) (layer F.Cu) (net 6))
 (segment (start 150.9 98) (end 150.9 99.0253) (width 0.25) (layer B.Cu) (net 6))
 (segment (start 164.338 123.825) (end 163.1491 123.825) (width 0.25) (layer B.Cu) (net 6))
 (segment (start 163.1491 123.825) (end 163.1491 111.2744) (width 0.25) (layer B.Cu) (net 6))
 (segment (start 163.1491 111.2744) (end 150.9 99.0253) (width 0.25) (layer B.Cu) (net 6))
 (segment (start 166.878 123.825) (end 166.878 114.3664) (width 0.25) (layer B.Cu) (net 3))
 (segment (start 166.878 114.3664) (end 152.691 100.1794) (width 0.25) (layer B.Cu) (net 3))
 (segment (start 152.691 100.1794) (end 152.691 97.0449) (width 0.25) (layer B.Cu) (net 3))
 (segment (start 152.691 97.0449) (end 148.9 93.2539) (width 0.25) (layer B.Cu) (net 3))
 (segment (start 148.9 93.2539) (end 148.9 89) (width 0.25) (layer B.Cu) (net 3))
 (segment (start 148.9 89) (end 149.9253 89) (width 0.25) (layer F.Cu) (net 3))
 (segment (start 152 88) (end 150.9253 88) (width 0.25) (layer F.Cu) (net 3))
 (segment (start 150.9253 88) (end 149.9253 89) (width 0.25) (layer F.Cu) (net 3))
 (segment (start 171.958 123.825) (end 171.958 118.3452) (width 0.25) (layer B.Cu) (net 21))
 (segment (start 171.958 118.3452) (end 153.1414 99.5286) (width 0.25) (layer B.Cu) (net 21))
 (segment (start 153.1414 99.5286) (end 153.1414 94.9258) (width 0.25) (layer B.Cu) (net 21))
 (segment (start 153.1414 94.9258) (end 150.2593 92.0437) (width 0.25) (layer B.Cu) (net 21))
 (segment (start 150.2593 92.0437) (end 150.2593 85.9046) (width 0.25) (layer B.Cu) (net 21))
 (segment (start 150.2593 85.9046) (end 145.96 81.6053) (width 0.25) (layer B.Cu) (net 21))
 (segment (start 145.96 81.6053) (end 144.1169 81.6053) (width 0.25) (layer B.Cu) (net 21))
 (segment (start 144.1169 81.6053) (end 138.684 76.1724) (width 0.25) (layer B.Cu) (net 21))
 (segment (start 138.684 76.1724) (end 138.684 74.9491) (width 0.25) (layer B.Cu) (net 21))
 (segment (start 138.684 74.9491) (end 137.9484 74.2135) (width 0.25) (layer B.Cu) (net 21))
 (segment (start 137.9484 74.2135) (end 134.3543 74.2135) (width 0.25) (layer B.Cu) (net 21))
 (segment (start 134.3543 74.2135) (end 133.5229 75.0449) (width 0.25) (layer B.Cu) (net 21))
 (segment (start 133.5229 75.0449) (end 133.5229 75.565) (width 0.25) (layer B.Cu) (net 21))
 (segment (start 132.334 75.565) (end 133.5229 75.565) (width 0.25) (layer B.Cu) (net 21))
 (segment (start 174.498 123.825) (end 174.498 120.2346) (width 0.25) (layer B.Cu) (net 22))
 (segment (start 174.498 120.2346) (end 154.0195 99.7561) (width 0.25) (layer B.Cu) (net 22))
 (segment (start 154.0195 99.7561) (end 154.0195 95.1669) (width 0.25) (layer B.Cu) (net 22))
 (segment (start 154.0195 95.1669) (end 150.725 91.8724) (width 0.25) (layer B.Cu) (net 22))
 (segment (start 150.725 91.8724) (end 150.725 85.651) (width 0.25) (layer B.Cu) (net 22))
 (segment (start 150.725 85.651) (end 141.2565 76.1825) (width 0.25) (layer B.Cu) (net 22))
 (segment (start 141.2565 76.1825) (end 141.2565 74.9941) (width 0.25) (layer B.Cu) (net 22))
 (segment (start 141.2565 74.9941) (end 140.0255 73.7631) (width 0.25) (layer B.Cu) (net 22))
 (segment (start 140.0255 73.7631) (end 132.2647 73.7631) (width 0.25) (layer B.Cu) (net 22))
 (segment (start 132.2647 73.7631) (end 130.9829 75.0449) (width 0.25) (layer B.Cu) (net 22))
 (segment (start 130.9829 75.0449) (end 130.9829 75.565) (width 0.25) (layer B.Cu) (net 22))
 (segment (start 129.794 75.565) (end 130.9829 75.565) (width 0.25) (layer B.Cu) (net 22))
 (segment (start 162 105.54) (end 160.9247 105.54) (width 0.25) (layer F.Cu) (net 7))
 (segment (start 160.9247 105.54) (end 160.31 104.9253) (width 0.25) (layer F.Cu) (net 7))
 (segment (start 160.31 104.9253) (end 155.0747 104.9253) (width 0.25) (layer F.Cu) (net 7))
 (segment (start 155.0747 104.9253) (end 154 106) (width 0.25) (layer F.Cu) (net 7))
 (segment (start 171 105) (end 170.46 105.54) (width 0.25) (layer B.Cu) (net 7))
 (segment (start 170.46 105.54) (end 162 105.54) (width 0.25) (layer B.Cu) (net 7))
 (segment (start 141 106) (end 144 103) (width 0.25) (layer F.Cu) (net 14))
 (segment (start 144 103) (end 144 100) (width 0.25) (layer F.Cu) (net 14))
 (segment (start 157.54 99) (end 157.54 100.0753) (width 0.25) (layer F.Cu) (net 5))
 (segment (start 149 106) (end 154.9247 100.0753) (width 0.25) (layer F.Cu) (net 5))
 (segment (start 154.9247 100.0753) (end 157.54 100.0753) (width 0.25) (layer F.Cu) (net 5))
 (segment (start 149 111) (end 149 106) (width 0.25) (layer B.Cu) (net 5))
 (segment (start 158.6952 91.3048) (end 158 92) (width 0.25) (layer F.Cu) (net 2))
 (segment (start 173 85) (end 167.3464 90.6536) (width 0.25) (layer F.Cu) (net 2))
 (segment (start 167.3464 90.6536) (end 159.3464 90.6536) (width 0.25) (layer F.Cu) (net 2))
 (segment (start 159.3464 90.6536) (end 158.6952 91.3048) (width 0.25) (layer F.Cu) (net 2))
 (segment (start 158.6952 91.3048) (end 155.3903 88) (width 0.25) (layer F.Cu) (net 2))
 (segment (start 154.54 88) (end 155.3903 88) (width 0.25) (layer F.Cu) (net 2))
 (segment (start 145 113) (end 145 112.2497) (width 0.25) (layer F.Cu) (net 13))
 (segment (start 145.0331 109.0331) (end 144 108) (width 0.25) (layer F.Cu) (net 13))
 (segment (start 162 104.27) (end 154.1927 104.27) (width 0.25) (layer F.Cu) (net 13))
 (segment (start 154.1927 104.27) (end 149.4296 109.0331) (width 0.25) (layer F.Cu) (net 13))
 (segment (start 149.4296 109.0331) (end 145.0331 109.0331) (width 0.25) (layer F.Cu) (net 13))
 (segment (start 145.0331 109.0331) (end 145.0331 112.2166) (width 0.25) (layer F.Cu) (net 13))
 (segment (start 145.0331 112.2166) (end 145 112.2497) (width 0.25) (layer F.Cu) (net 13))
 (segment (start 144 108) (end 142.1253 108) (width 0.25) (layer F.Cu) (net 13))
 (segment (start 142.1253 108) (end 142.0253 107.9) (width 0.25) (layer F.Cu) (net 13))
 (segment (start 141 107.9) (end 142.0253 107.9) (width 0.25) (layer F.Cu) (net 13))
 (segment (start 167 92) (end 166.2497 92) (width 0.25) (layer B.Cu) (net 11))
 (segment (start 166.2497 92) (end 166.2497 97.7503) (width 0.25) (layer B.Cu) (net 11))
 (segment (start 166.2497 97.7503) (end 166 98) (width 0.25) (layer B.Cu) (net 11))
 (segment (start 156.27 97.9247) (end 156.27 97.8059) (width 0.25) (layer F.Cu) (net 11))
 (segment (start 156.27 97.8059) (end 153.4641 95) (width 0.25) (layer F.Cu) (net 11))
 (segment (start 153.4641 95) (end 144.9 95) (width 0.25) (layer F.Cu) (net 11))
 (segment (start 156.27 99) (end 156.27 97.9247) (width 0.25) (layer F.Cu) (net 11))
 (segment (start 156.27 97.9247) (end 165.9247 97.9247) (width 0.25) (layer F.Cu) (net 11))
 (segment (start 165.9247 97.9247) (end 166 98) (width 0.25) (layer F.Cu) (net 11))
 (segment (start 144.9253 89) (end 147.0006 86.9247) (width 0.25) (layer F.Cu) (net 9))
 (segment (start 147.0006 86.9247) (end 153.27 86.9247) (width 0.25) (layer F.Cu) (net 9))
 (segment (start 143.9 89) (end 144.9253 89) (width 0.25) (layer F.Cu) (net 9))
 (segment (start 153.27 86.9247) (end 154.1947 86) (width 0.25) (layer F.Cu) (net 9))
 (segment (start 154.1947 86) (end 162 86) (width 0.25) (layer F.Cu) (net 9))
 (segment (start 153.27 88) (end 153.27 86.9247) (width 0.25) (layer F.Cu) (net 9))
 (segment (start 162 86) (end 162.7503 86) (width 0.25) (layer F.Cu) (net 9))
 (segment (start 162.7503 86) (end 163.7503 85) (width 0.25) (layer F.Cu) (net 9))
 (segment (start 163.7503 85) (end 168 85) (width 0.25) (layer F.Cu) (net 9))
 (segment (start 140 84) (end 140 92) (width 0.25) (layer B.Cu) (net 12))
 (segment (start 140 92) (end 143 95) (width 0.25) (layer B.Cu) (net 12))
 (segment (start 145 84) (end 142 87) (width 0.25) (layer B.Cu) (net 10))
 (segment (start 142 87) (end 142 89) (width 0.25) (layer B.Cu) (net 10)))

